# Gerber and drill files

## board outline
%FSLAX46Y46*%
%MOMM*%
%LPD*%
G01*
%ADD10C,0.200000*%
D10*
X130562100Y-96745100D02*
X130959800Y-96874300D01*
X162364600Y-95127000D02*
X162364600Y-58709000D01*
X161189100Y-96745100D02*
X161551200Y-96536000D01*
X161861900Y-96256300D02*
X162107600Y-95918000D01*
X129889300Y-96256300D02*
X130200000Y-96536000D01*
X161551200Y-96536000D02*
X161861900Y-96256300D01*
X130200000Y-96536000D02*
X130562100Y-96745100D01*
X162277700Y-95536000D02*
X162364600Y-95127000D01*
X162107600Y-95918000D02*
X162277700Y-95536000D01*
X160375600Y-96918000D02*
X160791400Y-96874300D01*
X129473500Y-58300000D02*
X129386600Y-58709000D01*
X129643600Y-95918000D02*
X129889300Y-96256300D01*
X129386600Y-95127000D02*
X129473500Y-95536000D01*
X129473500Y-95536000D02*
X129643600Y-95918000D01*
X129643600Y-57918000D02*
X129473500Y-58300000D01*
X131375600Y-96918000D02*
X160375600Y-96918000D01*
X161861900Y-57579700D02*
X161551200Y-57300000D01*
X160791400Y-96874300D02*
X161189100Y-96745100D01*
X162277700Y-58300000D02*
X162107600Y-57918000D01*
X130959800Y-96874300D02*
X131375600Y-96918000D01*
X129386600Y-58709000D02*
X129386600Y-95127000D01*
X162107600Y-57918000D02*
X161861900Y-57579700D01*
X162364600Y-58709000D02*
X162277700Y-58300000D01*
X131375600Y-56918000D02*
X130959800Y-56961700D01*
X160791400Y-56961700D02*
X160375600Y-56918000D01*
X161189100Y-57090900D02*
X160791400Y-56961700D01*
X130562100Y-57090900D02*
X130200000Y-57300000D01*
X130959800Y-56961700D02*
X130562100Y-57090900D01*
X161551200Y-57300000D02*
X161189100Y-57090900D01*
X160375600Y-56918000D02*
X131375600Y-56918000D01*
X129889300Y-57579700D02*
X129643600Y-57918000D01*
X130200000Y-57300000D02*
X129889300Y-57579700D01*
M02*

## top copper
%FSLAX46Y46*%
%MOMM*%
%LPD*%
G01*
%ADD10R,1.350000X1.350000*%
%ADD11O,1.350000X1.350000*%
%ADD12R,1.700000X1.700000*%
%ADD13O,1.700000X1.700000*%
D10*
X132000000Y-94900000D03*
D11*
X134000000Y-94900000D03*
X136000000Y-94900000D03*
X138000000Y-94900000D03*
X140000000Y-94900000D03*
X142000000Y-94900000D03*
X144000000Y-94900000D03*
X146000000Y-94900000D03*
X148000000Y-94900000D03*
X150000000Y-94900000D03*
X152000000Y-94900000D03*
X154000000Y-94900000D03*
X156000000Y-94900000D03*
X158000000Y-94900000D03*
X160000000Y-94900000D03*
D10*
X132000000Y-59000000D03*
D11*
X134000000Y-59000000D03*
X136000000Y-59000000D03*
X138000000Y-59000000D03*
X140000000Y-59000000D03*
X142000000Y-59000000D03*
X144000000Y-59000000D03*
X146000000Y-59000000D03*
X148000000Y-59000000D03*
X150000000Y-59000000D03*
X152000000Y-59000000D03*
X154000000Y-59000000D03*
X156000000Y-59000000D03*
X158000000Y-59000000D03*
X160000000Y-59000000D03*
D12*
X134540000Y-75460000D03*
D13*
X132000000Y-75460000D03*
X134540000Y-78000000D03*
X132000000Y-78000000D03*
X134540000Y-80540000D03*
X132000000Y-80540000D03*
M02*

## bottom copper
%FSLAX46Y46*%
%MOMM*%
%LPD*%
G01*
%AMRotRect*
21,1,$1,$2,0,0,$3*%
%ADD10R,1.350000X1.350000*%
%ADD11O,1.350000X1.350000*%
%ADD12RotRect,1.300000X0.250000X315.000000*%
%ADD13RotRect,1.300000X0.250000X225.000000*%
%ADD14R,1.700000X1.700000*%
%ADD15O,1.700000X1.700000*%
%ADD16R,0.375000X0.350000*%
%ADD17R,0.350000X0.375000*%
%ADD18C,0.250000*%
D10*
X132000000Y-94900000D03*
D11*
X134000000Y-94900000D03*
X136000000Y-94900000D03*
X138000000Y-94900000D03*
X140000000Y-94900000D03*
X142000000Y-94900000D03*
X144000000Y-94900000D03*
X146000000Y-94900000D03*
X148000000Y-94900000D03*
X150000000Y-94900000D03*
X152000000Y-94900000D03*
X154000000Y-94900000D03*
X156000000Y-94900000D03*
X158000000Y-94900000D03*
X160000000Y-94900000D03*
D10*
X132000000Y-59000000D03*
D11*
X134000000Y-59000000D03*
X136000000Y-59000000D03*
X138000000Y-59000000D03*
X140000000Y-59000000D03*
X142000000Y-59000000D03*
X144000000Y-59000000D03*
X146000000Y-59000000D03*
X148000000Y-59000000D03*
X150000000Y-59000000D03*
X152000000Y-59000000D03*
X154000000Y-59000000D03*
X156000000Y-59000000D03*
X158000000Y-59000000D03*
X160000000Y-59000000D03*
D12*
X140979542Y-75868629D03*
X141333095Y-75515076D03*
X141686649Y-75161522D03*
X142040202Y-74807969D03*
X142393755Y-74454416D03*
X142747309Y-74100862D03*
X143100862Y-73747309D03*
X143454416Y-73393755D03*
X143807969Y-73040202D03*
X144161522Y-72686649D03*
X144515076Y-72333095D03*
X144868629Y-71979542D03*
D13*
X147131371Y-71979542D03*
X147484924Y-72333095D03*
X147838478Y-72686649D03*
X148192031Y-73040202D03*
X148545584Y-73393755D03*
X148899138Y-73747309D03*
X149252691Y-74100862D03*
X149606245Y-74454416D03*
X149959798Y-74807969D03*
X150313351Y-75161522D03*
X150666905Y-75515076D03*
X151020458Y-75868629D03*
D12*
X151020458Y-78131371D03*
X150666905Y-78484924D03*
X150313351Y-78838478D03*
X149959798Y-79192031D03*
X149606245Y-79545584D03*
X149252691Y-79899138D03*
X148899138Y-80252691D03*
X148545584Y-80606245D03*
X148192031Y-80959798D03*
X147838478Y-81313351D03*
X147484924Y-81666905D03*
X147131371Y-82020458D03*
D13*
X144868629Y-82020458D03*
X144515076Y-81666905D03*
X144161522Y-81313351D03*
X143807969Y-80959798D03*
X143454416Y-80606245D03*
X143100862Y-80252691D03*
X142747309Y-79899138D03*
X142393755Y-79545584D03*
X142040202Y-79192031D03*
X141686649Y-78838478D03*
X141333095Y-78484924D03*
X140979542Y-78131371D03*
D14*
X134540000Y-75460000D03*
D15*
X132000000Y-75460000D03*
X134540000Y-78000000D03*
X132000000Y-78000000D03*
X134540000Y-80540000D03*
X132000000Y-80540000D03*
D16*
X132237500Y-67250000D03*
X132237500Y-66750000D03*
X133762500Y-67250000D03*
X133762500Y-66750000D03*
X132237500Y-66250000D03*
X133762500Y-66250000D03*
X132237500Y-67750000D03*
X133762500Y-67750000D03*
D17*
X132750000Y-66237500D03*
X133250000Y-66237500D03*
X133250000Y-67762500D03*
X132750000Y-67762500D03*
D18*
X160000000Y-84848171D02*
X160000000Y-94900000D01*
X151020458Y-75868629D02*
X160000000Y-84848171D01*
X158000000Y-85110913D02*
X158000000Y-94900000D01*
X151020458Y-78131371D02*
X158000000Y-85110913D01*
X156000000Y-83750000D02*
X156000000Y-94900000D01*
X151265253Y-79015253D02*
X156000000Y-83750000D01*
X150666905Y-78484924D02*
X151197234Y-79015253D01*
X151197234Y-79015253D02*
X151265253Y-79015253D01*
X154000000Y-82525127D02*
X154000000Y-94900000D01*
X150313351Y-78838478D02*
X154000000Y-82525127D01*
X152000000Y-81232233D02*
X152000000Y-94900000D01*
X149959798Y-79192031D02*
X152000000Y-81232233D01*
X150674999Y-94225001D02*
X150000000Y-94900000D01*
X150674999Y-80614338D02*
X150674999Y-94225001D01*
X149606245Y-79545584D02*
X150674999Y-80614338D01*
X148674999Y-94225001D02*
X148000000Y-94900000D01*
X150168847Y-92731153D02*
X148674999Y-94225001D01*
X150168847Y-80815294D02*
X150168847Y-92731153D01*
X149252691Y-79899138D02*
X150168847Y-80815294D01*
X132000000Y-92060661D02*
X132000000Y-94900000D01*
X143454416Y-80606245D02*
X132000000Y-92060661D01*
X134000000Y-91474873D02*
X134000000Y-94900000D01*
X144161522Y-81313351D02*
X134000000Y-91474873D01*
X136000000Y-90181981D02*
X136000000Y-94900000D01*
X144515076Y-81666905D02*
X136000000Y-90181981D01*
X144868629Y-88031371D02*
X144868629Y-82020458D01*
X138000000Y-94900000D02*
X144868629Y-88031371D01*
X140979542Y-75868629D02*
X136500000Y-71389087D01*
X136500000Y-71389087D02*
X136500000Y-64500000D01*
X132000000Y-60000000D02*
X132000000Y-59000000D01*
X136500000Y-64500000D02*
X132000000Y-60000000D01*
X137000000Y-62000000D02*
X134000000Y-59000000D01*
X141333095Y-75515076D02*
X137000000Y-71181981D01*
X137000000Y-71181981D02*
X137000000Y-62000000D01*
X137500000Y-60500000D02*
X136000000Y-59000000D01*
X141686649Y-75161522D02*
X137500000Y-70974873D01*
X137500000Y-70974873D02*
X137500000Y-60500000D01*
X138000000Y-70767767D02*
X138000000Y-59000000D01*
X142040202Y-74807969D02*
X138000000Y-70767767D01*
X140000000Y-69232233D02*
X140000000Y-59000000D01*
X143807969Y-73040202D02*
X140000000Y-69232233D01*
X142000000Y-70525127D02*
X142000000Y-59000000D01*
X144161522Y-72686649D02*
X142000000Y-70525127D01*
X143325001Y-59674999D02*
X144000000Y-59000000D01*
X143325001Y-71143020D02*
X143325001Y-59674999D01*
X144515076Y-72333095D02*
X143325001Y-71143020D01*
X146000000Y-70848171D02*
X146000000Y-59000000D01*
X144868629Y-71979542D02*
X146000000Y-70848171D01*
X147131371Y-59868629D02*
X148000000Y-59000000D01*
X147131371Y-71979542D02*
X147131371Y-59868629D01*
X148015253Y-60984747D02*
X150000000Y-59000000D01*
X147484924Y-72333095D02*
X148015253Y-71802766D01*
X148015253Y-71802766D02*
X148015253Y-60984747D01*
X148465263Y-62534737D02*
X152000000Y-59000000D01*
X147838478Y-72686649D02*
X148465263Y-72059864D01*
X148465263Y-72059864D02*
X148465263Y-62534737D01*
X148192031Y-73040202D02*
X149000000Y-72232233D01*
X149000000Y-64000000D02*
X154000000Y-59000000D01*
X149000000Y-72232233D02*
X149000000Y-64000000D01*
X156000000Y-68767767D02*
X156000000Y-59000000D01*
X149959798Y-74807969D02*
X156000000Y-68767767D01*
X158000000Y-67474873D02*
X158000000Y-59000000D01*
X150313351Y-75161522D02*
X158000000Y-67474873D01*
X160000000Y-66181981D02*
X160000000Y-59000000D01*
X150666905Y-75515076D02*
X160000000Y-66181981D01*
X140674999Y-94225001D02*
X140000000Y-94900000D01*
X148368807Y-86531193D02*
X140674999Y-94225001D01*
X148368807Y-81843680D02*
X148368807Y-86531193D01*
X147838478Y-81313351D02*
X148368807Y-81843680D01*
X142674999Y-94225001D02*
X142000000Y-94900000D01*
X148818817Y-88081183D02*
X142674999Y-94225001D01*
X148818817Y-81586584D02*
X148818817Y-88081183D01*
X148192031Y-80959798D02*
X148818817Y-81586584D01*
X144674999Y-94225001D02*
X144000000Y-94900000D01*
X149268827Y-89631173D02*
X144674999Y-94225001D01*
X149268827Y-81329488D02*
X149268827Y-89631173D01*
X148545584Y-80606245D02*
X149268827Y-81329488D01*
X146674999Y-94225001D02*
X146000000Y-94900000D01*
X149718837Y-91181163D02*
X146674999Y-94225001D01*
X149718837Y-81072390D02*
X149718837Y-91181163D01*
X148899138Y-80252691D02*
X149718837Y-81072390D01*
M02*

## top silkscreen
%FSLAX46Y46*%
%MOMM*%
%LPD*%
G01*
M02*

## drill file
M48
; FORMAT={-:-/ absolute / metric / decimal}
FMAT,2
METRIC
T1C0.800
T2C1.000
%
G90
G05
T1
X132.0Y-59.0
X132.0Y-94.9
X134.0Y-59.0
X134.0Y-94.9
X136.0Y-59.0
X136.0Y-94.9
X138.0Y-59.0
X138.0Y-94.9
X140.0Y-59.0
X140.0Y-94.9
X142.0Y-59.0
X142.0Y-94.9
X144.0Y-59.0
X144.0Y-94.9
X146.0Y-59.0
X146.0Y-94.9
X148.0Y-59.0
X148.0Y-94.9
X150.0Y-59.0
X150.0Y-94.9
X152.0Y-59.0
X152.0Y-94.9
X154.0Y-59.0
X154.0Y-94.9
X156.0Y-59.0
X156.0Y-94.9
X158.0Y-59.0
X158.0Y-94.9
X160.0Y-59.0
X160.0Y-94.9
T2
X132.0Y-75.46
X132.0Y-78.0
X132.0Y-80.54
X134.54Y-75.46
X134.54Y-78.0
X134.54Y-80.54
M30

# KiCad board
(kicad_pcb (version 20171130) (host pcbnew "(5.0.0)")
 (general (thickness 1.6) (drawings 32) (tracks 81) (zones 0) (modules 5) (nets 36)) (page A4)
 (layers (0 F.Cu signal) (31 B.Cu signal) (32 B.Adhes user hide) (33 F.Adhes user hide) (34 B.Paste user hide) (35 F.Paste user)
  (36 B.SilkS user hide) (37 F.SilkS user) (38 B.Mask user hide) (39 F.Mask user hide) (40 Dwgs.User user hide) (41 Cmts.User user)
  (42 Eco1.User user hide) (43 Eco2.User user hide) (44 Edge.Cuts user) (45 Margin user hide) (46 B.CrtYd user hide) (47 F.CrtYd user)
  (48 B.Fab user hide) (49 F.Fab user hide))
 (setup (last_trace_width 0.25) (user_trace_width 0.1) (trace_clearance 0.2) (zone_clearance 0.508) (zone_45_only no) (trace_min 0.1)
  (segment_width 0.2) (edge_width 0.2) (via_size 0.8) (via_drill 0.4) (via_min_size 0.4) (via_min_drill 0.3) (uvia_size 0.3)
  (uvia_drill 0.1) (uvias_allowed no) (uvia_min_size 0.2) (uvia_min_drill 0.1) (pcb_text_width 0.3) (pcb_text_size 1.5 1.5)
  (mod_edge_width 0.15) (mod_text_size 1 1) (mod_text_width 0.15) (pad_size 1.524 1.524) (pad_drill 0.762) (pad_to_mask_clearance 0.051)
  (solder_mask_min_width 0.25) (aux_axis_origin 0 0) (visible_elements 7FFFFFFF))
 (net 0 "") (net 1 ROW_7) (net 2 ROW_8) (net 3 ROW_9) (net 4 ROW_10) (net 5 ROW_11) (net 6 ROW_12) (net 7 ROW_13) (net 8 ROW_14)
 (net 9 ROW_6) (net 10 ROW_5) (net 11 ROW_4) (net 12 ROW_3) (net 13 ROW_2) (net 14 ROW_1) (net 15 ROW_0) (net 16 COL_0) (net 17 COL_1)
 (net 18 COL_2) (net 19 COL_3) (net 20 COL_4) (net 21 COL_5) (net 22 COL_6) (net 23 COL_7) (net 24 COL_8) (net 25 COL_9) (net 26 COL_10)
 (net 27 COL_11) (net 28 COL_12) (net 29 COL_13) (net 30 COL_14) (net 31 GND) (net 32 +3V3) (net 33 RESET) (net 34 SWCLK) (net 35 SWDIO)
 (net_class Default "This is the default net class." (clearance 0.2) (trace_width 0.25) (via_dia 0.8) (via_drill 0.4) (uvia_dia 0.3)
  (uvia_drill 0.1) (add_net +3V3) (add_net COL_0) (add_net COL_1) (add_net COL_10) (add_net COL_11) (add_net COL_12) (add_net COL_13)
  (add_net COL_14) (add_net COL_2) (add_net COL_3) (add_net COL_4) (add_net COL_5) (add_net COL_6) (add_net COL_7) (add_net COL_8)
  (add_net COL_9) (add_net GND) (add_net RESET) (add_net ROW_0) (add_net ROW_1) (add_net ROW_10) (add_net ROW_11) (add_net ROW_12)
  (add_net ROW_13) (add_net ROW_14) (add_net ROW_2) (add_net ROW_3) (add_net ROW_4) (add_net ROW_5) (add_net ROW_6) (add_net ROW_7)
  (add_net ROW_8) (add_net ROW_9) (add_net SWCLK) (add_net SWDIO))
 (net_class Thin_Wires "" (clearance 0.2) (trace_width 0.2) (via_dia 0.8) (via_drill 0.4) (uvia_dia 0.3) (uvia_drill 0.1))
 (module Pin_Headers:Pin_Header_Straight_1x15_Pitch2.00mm (layer F.Cu) (at 132 94.9 90)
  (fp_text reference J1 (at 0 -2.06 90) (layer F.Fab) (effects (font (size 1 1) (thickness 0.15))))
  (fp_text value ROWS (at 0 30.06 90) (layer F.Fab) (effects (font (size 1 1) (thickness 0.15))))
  (pad 1 thru_hole rect (at 0 0 90) (size 1.35 1.35) (drill 0.8) (layers *.Cu *.Mask) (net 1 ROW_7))
  (pad 2 thru_hole oval (at 0 2 90) (size 1.35 1.35) (drill 0.8) (layers *.Cu *.Mask) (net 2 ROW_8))
  (pad 3 thru_hole oval (at 0 4 90) (size 1.35 1.35) (drill 0.8) (layers *.Cu *.Mask) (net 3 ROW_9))
  (pad 4 thru_hole oval (at 0 6 90) (size 1.35 1.35) (drill 0.8) (layers *.Cu *.Mask) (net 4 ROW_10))
  (pad 5 thru_hole oval (at 0 8 90) (size 1.35 1.35) (drill 0.8) (layers *.Cu *.Mask) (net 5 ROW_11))
  (pad 6 thru_hole oval (at 0 10 90) (size 1.35 1.35) (drill 0.8) (layers *.Cu *.Mask) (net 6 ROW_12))
  (pad 7 thru_hole oval (at 0 12 90) (size 1.35 1.35) (drill 0.8) (layers *.Cu *.Mask) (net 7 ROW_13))
  (pad 8 thru_hole oval (at 0 14 90) (size 1.35 1.35) (drill 0.8) (layers *.Cu *.Mask) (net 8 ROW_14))
  (pad 9 thru_hole oval (at 0 16 90) (size 1.35 1.35) (drill 0.8) (layers *.Cu *.Mask) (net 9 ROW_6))
  (pad 10 thru_hole oval (at 0 18 90) (size 1.35 1.35) (drill 0.8) (layers *.Cu *.Mask) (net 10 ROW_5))
  (pad 11 thru_hole oval (at 0 20 90) (size 1.35 1.35) (drill 0.8) (layers *.Cu *.Mask) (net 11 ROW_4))
  (pad 12 thru_hole oval (at 0 22 90) (size 1.35 1.35) (drill 0.8) (layers *.Cu *.Mask) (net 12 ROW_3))
  (pad 13 thru_hole oval (at 0 24 90) (size 1.35 1.35) (drill 0.8) (layers *.Cu *.Mask) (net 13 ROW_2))
  (pad 14 thru_hole oval (at 0 26 90) (size 1.35 1.35) (drill 0.8) (layers *.Cu *.Mask) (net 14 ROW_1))
  (pad 15 thru_hole oval (at 0 28 90) (size 1.35 1.35) (drill 0.8) (layers *.Cu *.Mask) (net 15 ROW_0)))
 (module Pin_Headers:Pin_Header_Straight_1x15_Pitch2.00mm (layer F.Cu) (at 132 59 90)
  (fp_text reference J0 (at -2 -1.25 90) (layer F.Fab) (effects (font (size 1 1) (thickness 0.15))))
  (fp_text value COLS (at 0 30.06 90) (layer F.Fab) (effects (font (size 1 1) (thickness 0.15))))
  (pad 1 thru_hole rect (at 0 0 90) (size 1.35 1.35) (drill 0.8) (layers *.Cu *.Mask) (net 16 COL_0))
  (pad 2 thru_hole oval (at 0 2 90) (size 1.35 1.35) (drill 0.8) (layers *.Cu *.Mask) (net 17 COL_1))
  (pad 3 thru_hole oval (at 0 4 90) (size 1.35 1.35) (drill 0.8) (layers *.Cu *.Mask) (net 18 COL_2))
  (pad 4 thru_hole oval (at 0 6 90) (size 1.35 1.35) (drill 0.8) (layers *.Cu *.Mask) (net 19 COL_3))
  (pad 5 thru_hole oval (at 0 8 90) (size 1.35 1.35) (drill 0.8) (layers *.Cu *.Mask) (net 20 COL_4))
  (pad 6 thru_hole oval (at 0 10 90) (size 1.35 1.35) (drill 0.8) (layers *.Cu *.Mask) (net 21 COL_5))
  (pad 7 thru_hole oval (at 0 12 90) (size 1.35 1.35) (drill 0.8) (layers *.Cu *.Mask) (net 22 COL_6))
  (pad 8 thru_hole oval (at 0 14 90) (size 1.35 1.35) (drill 0.8) (layers *.Cu *.Mask) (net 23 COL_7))
  (pad 9 thru_hole oval (at 0 16 90) (size 1.35 1.35) (drill 0.8) (layers *.Cu *.Mask) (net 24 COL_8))
  (pad 10 thru_hole oval (at 0 18 90) (size 1.35 1.35) (drill 0.8) (layers *.Cu *.Mask) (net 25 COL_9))
  (pad 11 thru_hole oval (at 0 20 90) (size 1.35 1.35) (drill 0.8) (layers *.Cu *.Mask) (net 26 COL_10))
  (pad 12 thru_hole oval (at 0 22 90) (size 1.35 1.35) (drill 0.8) (layers *.Cu *.Mask) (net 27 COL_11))
  (pad 13 thru_hole oval (at 0 24 90) (size 1.35 1.35) (drill 0.8) (layers *.Cu *.Mask) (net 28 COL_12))
  (pad 14 thru_hole oval (at 0 26 90) (size 1.35 1.35) (drill 0.8) (layers *.Cu *.Mask) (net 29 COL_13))
  (pad 15 thru_hole oval (at 0 28 90) (size 1.35 1.35) (drill 0.8) (layers *.Cu *.Mask) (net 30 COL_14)))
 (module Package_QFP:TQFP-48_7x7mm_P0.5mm (layer B.Cu) (at 146 77 315)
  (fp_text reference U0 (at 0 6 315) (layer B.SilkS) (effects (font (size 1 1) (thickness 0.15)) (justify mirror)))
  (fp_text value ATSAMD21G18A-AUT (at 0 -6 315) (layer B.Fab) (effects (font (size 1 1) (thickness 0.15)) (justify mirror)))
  (pad 1 smd rect (at -4.35 2.75 315) (size 1.3 0.25) (layers B.Cu B.Paste B.Mask) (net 16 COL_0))
  (pad 2 smd rect (at -4.35 2.25 315) (size 1.3 0.25) (layers B.Cu B.Paste B.Mask) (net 17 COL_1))
  (pad 3 smd rect (at -4.35 1.749999 315) (size 1.3 0.25) (layers B.Cu B.Paste B.Mask) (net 18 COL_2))
  (pad 4 smd rect (at -4.35 1.25 315) (size 1.3 0.25) (layers B.Cu B.Paste B.Mask) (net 19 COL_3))
  (pad 5 smd rect (at -4.35 0.750001 315) (size 1.3 0.25) (layers B.Cu B.Paste B.Mask) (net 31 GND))
  (pad 6 smd rect (at -4.35 0.25 315) (size 1.3 0.25) (layers B.Cu B.Paste B.Mask) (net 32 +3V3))
  (pad 7 smd rect (at -4.35 -0.25 315) (size 1.3 0.25) (layers B.Cu B.Paste B.Mask))
  (pad 8 smd rect (at -4.35 -0.750001 315) (size 1.3 0.25) (layers B.Cu B.Paste B.Mask))
  (pad 9 smd rect (at -4.35 -1.25 315) (size 1.3 0.25) (layers B.Cu B.Paste B.Mask) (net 20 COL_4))
  (pad 10 smd rect (at -4.35 -1.749999 315) (size 1.3 0.25) (layers B.Cu B.Paste B.Mask) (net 21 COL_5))
  (pad 11 smd rect (at -4.35 -2.25 315) (size 1.3 0.25) (layers B.Cu B.Paste B.Mask) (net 22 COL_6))
  (pad 12 smd rect (at -4.35 -2.75 315) (size 1.3 0.25) (layers B.Cu B.Paste B.Mask) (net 23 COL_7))
  (pad 13 smd rect (at -2.75 -4.35 225) (size 1.3 0.25) (layers B.Cu B.Paste B.Mask) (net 24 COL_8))
  (pad 14 smd rect (at -2.25 -4.35 225) (size 1.3 0.25) (layers B.Cu B.Paste B.Mask) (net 25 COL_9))
  (pad 15 smd rect (at -1.749999 -4.35 225) (size 1.3 0.25) (layers B.Cu B.Paste B.Mask) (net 26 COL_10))
  (pad 16 smd rect (at -1.25 -4.35 225) (size 1.3 0.25) (layers B.Cu B.Paste B.Mask) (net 27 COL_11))
  (pad 17 smd rect (at -0.750001 -4.35 225) (size 1.3 0.25) (layers B.Cu B.Paste B.Mask) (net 32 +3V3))
  (pad 18 smd rect (at -0.25 -4.35 225) (size 1.3 0.25) (layers B.Cu B.Paste B.Mask) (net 31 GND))
  (pad 19 smd rect (at 0.25 -4.35 225) (size 1.3 0.25) (layers B.Cu B.Paste B.Mask))
  (pad 20 smd rect (at 0.750001 -4.35 225) (size 1.3 0.25) (layers B.Cu B.Paste B.Mask))
  (pad 21 smd rect (at 1.25 -4.35 225) (size 1.3 0.25) (layers B.Cu B.Paste B.Mask) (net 28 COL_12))
  (pad 22 smd rect (at 1.749999 -4.35 225) (size 1.3 0.25) (layers B.Cu B.Paste B.Mask) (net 29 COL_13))
  (pad 23 smd rect (at 2.25 -4.35 225) (size 1.3 0.25) (layers B.Cu B.Paste B.Mask) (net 30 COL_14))
  (pad 24 smd rect (at 2.75 -4.35 225) (size 1.3 0.25) (layers B.Cu B.Paste B.Mask) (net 15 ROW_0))
  (pad 25 smd rect (at 4.35 -2.75 315) (size 1.3 0.25) (layers B.Cu B.Paste B.Mask) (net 14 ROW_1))
  (pad 26 smd rect (at 4.35 -2.25 315) (size 1.3 0.25) (layers B.Cu B.Paste B.Mask) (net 13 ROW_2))
  (pad 27 smd rect (at 4.35 -1.749999 315) (size 1.3 0.25) (layers B.Cu B.Paste B.Mask) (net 12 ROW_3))
  (pad 28 smd rect (at 4.35 -1.25 315) (size 1.3 0.25) (layers B.Cu B.Paste B.Mask) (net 11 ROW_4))
  (pad 29 smd rect (at 4.35 -0.750001 315) (size 1.3 0.25) (layers B.Cu B.Paste B.Mask) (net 10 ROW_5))
  (pad 30 smd rect (at 4.35 -0.25 315) (size 1.3 0.25) (layers B.Cu B.Paste B.Mask) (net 9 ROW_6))
  (pad 31 smd rect (at 4.35 0.25 315) (size 1.3 0.25) (layers B.Cu B.Paste B.Mask) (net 8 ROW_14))
  (pad 32 smd rect (at 4.35 0.750001 315) (size 1.3 0.25) (layers B.Cu B.Paste B.Mask) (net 7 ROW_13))
  (pad 33 smd rect (at 4.35 1.25 315) (size 1.3 0.25) (layers B.Cu B.Paste B.Mask) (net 6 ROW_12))
  (pad 34 smd rect (at 4.35 1.749999 315) (size 1.3 0.25) (layers B.Cu B.Paste B.Mask) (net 5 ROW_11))
  (pad 35 smd rect (at 4.35 2.25 315) (size 1.3 0.25) (layers B.Cu B.Paste B.Mask) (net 31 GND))
  (pad 36 smd rect (at 4.35 2.75 315) (size 1.3 0.25) (layers B.Cu B.Paste B.Mask) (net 32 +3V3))
  (pad 37 smd rect (at 2.75 4.35 225) (size 1.3 0.25) (layers B.Cu B.Paste B.Mask) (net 4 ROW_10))
  (pad 38 smd rect (at 2.25 4.35 225) (size 1.3 0.25) (layers B.Cu B.Paste B.Mask) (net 3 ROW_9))
  (pad 39 smd rect (at 1.749999 4.35 225) (size 1.3 0.25) (layers B.Cu B.Paste B.Mask) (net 2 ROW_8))
  (pad 40 smd rect (at 1.25 4.35 225) (size 1.3 0.25) (layers B.Cu B.Paste B.Mask) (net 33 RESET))
  (pad 41 smd rect (at 0.750001 4.35 225) (size 1.3 0.25) (layers B.Cu B.Paste B.Mask) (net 1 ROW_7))
  (pad 42 smd rect (at 0.25 4.35 225) (size 1.3 0.25) (layers B.Cu B.Paste B.Mask) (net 31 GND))
  (pad 43 smd rect (at -0.25 4.35 225) (size 1.3 0.25) (layers B.Cu B.Paste B.Mask) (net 32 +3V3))
  (pad 44 smd rect (at -0.750001 4.35 225) (size 1.3 0.25) (layers B.Cu B.Paste B.Mask) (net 32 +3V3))
  (pad 45 smd rect (at -1.25 4.35 225) (size 1.3 0.25) (layers B.Cu B.Paste B.Mask) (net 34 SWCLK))
  (pad 46 smd rect (at -1.749999 4.35 225) (size 1.3 0.25) (layers B.Cu B.Paste B.Mask) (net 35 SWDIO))
  (pad 47 smd rect (at -2.25 4.35 225) (size 1.3 0.25) (layers B.Cu B.Paste B.Mask))
  (pad 48 smd rect (at -2.75 4.35 225) (size 1.3 0.25) (layers B.Cu B.Paste B.Mask)))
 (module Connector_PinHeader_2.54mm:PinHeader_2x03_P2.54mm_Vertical (layer B.Cu) (at 134.54 75.46 180)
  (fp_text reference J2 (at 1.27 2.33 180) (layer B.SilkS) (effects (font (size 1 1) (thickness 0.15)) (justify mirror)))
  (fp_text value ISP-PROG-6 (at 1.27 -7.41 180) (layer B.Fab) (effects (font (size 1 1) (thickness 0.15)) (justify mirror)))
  (pad 1 thru_hole rect (at 0 0 180) (size 1.7 1.7) (drill 1) (layers *.Cu *.Mask) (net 35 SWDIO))
  (pad 2 thru_hole oval (at 2.54 0 180) (size 1.7 1.7) (drill 1) (layers *.Cu *.Mask) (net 32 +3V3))
  (pad 3 thru_hole oval (at 0 -2.54 180) (size 1.7 1.7) (drill 1) (layers *.Cu *.Mask) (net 34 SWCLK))
  (pad 4 thru_hole oval (at 2.54 -2.54 180) (size 1.7 1.7) (drill 1) (layers *.Cu *.Mask))
  (pad 5 thru_hole oval (at 0 -5.08 180) (size 1.7 1.7) (drill 1) (layers *.Cu *.Mask) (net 33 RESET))
  (pad 6 thru_hole oval (at 2.54 -5.08 180) (size 1.7 1.7) (drill 1) (layers *.Cu *.Mask) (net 31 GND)))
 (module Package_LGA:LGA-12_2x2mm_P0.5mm (layer B.Cu) (at 133 67)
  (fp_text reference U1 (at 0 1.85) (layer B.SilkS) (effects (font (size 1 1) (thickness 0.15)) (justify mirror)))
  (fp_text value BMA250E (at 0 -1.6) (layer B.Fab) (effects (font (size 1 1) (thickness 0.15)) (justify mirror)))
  (pad 2 smd rect (at -0.7625 0.25) (size 0.375 0.35) (layers B.Cu B.Paste B.Mask))
  (pad 3 smd rect (at -0.7625 -0.25) (size 0.375 0.35) (layers B.Cu B.Paste B.Mask))
  (pad 9 smd rect (at 0.7625 0.25) (size 0.375 0.35) (layers B.Cu B.Paste B.Mask))
  (pad 8 smd rect (at 0.7625 -0.25) (size 0.375 0.35) (layers B.Cu B.Paste B.Mask))
  (pad 4 smd rect (at -0.7625 -0.75) (size 0.375 0.35) (layers B.Cu B.Paste B.Mask))
  (pad 7 smd rect (at 0.7625 -0.75) (size 0.375 0.35) (layers B.Cu B.Paste B.Mask))
  (pad 1 smd rect (at -0.7625 0.75) (size 0.375 0.35) (layers B.Cu B.Paste B.Mask))
  (pad 10 smd rect (at 0.7625 0.75) (size 0.375 0.35) (layers B.Cu B.Paste B.Mask))
  (pad 5 smd rect (at -0.25 -0.7625 270) (size 0.375 0.35) (layers B.Cu B.Paste B.Mask))
  (pad 6 smd rect (at 0.25 -0.7625 270) (size 0.375 0.35) (layers B.Cu B.Paste B.Mask))
  (pad 11 smd rect (at 0.25 0.7625 270) (size 0.375 0.35) (layers B.Cu B.Paste B.Mask))
  (pad 12 smd rect (at -0.25 0.7625 270) (size 0.375 0.35) (layers B.Cu B.Paste B.Mask)))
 (gr_line (start 130.5621 96.7451) (end 130.9598 96.8743) (layer Edge.Cuts) (width 0.2))
 (gr_line (start 162.3646 95.127) (end 162.3646 58.709) (layer Edge.Cuts) (width 0.2))
 (gr_line (start 161.1891 96.7451) (end 161.5512 96.536) (layer Edge.Cuts) (width 0.2))
 (gr_line (start 161.8619 96.2563) (end 162.1076 95.918) (layer Edge.Cuts) (width 0.2))
 (gr_line (start 129.8893 96.2563) (end 130.2 96.536) (layer Edge.Cuts) (width 0.2))
 (gr_line (start 161.5512 96.536) (end 161.8619 96.2563) (layer Edge.Cuts) (width 0.2))
 (gr_line (start 130.2 96.536) (end 130.5621 96.7451) (layer Edge.Cuts) (width 0.2))
 (gr_line (start 162.2777 95.536) (end 162.3646 95.127) (layer Edge.Cuts) (width 0.2))
 (gr_line (start 162.1076 95.918) (end 162.2777 95.536) (layer Edge.Cuts) (width 0.2))
 (gr_line (start 160.3756 96.918) (end 160.7914 96.8743) (layer Edge.Cuts) (width 0.2))
 (gr_line (start 129.4735 58.3) (end 129.3866 58.709) (layer Edge.Cuts) (width 0.2))
 (gr_line (start 129.6436 95.918) (end 129.8893 96.2563) (layer Edge.Cuts) (width 0.2))
 (gr_line (start 129.3866 95.127) (end 129.4735 95.536) (layer Edge.Cuts) (width 0.2))
 (gr_line (start 129.4735 95.536) (end 129.6436 95.918) (layer Edge.Cuts) (width 0.2))
 (gr_line (start 129.6436 57.918) (end 129.4735 58.3) (layer Edge.Cuts) (width 0.2))
 (gr_line (start 131.3756 96.918) (end 160.3756 96.918) (layer Edge.Cuts) (width 0.2))
 (gr_line (start 161.8619 57.5797) (end 161.5512 57.3) (layer Edge.Cuts) (width 0.2))
 (gr_line (start 160.7914 96.8743) (end 161.1891 96.7451) (layer Edge.Cuts) (width 0.2))
 (gr_line (start 162.2777 58.3) (end 162.1076 57.918) (layer Edge.Cuts) (width 0.2))
 (gr_line (start 130.9598 96.8743) (end 131.3756 96.918) (layer Edge.Cuts) (width 0.2))
 (gr_line (start 129.3866 58.709) (end 129.3866 95.127) (layer Edge.Cuts) (width 0.2))
 (gr_line (start 162.1076 57.918) (end 161.8619 57.5797) (layer Edge.Cuts) (width 0.2))
 (gr_line (start 162.3646 58.709) (end 162.2777 58.3) (layer Edge.Cuts) (width 0.2))
 (gr_line (start 131.3756 56.918) (end 130.9598 56.9617) (layer Edge.Cuts) (width 0.2))
 (gr_line (start 160.7914 56.9617) (end 160.3756 56.918) (layer Edge.Cuts) (width 0.2))
 (gr_line (start 161.1891 57.0909) (end 160.7914 56.9617) (layer Edge.Cuts) (width 0.2))
 (gr_line (start 130.5621 57.0909) (end 130.2 57.3) (layer Edge.Cuts) (width 0.2))
 (gr_line (start 130.9598 56.9617) (end 130.5621 57.0909) (layer Edge.Cuts) (width 0.2))
 (gr_line (start 161.5512 57.3) (end 161.1891 57.0909) (layer Edge.Cuts) (width 0.2))
 (gr_line (start 160.3756 56.918) (end 131.3756 56.918) (layer Edge.Cuts) (width 0.2))
 (gr_line (start 129.8893 57.5797) (end 129.6436 57.918) (layer Edge.Cuts) (width 0.2))
 (gr_line (start 130.2 57.3) (end 129.8893 57.5797) (layer Edge.Cuts) (width 0.2))
 (segment (start 160 84.848171) (end 160 94.9) (width 0.25) (layer B.Cu) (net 15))
 (segment (start 151.020458 75.868629) (end 160 84.848171) (width 0.25) (layer B.Cu) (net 15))
 (segment (start 158 85.110913) (end 158 94.9) (width 0.25) (layer B.Cu) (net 14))
 (segment (start 151.020458 78.131371) (end 158 85.110913) (width 0.25) (layer B.Cu) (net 14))
 (segment (start 156 83.75) (end 156 94.9) (width 0.25) (layer B.Cu) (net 13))
 (segment (start 151.265253 79.015253) (end 156 83.75) (width 0.25) (layer B.Cu) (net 13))
 (segment (start 150.666905 78.484924) (end 151.197234 79.015253) (width 0.25) (layer B.Cu) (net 13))
 (segment (start 151.197234 79.015253) (end 151.265253 79.015253) (width 0.25) (layer B.Cu) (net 13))
 (segment (start 154 82.525127) (end 154 94.9) (width 0.25) (layer B.Cu) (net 12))
 (segment (start 150.313351 78.838478) (end 154 82.525127) (width 0.25) (layer B.Cu) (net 12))
 (segment (start 152 81.232233) (end 152 94.9) (width 0.25) (layer B.Cu) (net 11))
 (segment (start 149.959798 79.192031) (end 152 81.232233) (width 0.25) (layer B.Cu) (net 11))
 (segment (start 150.674999 94.225001) (end 150 94.9) (width 0.25) (layer B.Cu) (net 10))
 (segment (start 150.674999 80.614338) (end 150.674999 94.225001) (width 0.25) (layer B.Cu) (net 10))
 (segment (start 149.606245 79.545584) (end 150.674999 80.614338) (width 0.25) (layer B.Cu) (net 10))
 (segment (start 148.674999 94.225001) (end 148 94.9) (width 0.25) (layer B.Cu) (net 9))
 (segment (start 150.168847 92.731153) (end 148.674999 94.225001) (width 0.25) (layer B.Cu) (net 9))
 (segment (start 150.168847 80.815294) (end 150.168847 92.731153) (width 0.25) (layer B.Cu) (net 9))
 (segment (start 149.252691 79.899138) (end 150.168847 80.815294) (width 0.25) (layer B.Cu) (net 9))
 (segment (start 132 92.060661) (end 132 94.9) (width 0.25) (layer B.Cu) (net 1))
 (segment (start 143.454416 80.606245) (end 132 92.060661) (width 0.25) (layer B.Cu) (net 1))
 (segment (start 134 91.474873) (end 134 94.9) (width 0.25) (layer B.Cu) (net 2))
 (segment (start 144.161522 81.313351) (end 134 91.474873) (width 0.25) (layer B.Cu) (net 2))
 (segment (start 136 90.181981) (end 136 94.9) (width 0.25) (layer B.Cu) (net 3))
 (segment (start 144.515076 81.666905) (end 136 90.181981) (width 0.25) (layer B.Cu) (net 3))
 (segment (start 144.868629 88.031371) (end 144.868629 82.020458) (width 0.25) (layer B.Cu) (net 4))
 (segment (start 138 94.9) (end 144.868629 88.031371) (width 0.25) (layer B.Cu) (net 4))
 (segment (start 140.979542 75.868629) (end 136.5 71.389087) (width 0.25) (layer B.Cu) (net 16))
 (segment (start 136.5 71.389087) (end 136.5 64.5) (width 0.25) (layer B.Cu) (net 16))
 (segment (start 132 60) (end 132 59) (width 0.25) (layer B.Cu) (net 16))
 (segment (start 136.5 64.5) (end 132 60) (width 0.25) (layer B.Cu) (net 16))
 (segment (start 137 62) (end 134 59) (width 0.25) (layer B.Cu) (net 17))
 (segment (start 141.333095 75.515076) (end 137 71.181981) (width 0.25) (layer B.Cu) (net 17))
 (segment (start 137 71.181981) (end 137 62) (width 0.25) (layer B.Cu) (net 17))
 (segment (start 137.5 60.5) (end 136 59) (width 0.25) (layer B.Cu) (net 18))
 (segment (start 141.686649 75.161522) (end 137.5 70.974873) (width 0.25) (layer B.Cu) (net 18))
 (segment (start 137.5 70.974873) (end 137.5 60.5) (width 0.25) (layer B.Cu) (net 18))
 (segment (start 138 70.767767) (end 138 59) (width 0.25) (layer B.Cu) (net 19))
 (segment (start 142.040202 74.807969) (end 138 70.767767) (width 0.25) (layer B.Cu) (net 19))
 (segment (start 140 69.232233) (end 140 59) (width 0.25) (layer B.Cu) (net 20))
 (segment (start 143.807969 73.040202) (end 140 69.232233) (width 0.25) (layer B.Cu) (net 20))
 (segment (start 142 70.525127) (end 142 59) (width 0.25) (layer B.Cu) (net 21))
 (segment (start 144.161522 72.686649) (end 142 70.525127) (width 0.25) (layer B.Cu) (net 21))
 (segment (start 143.325001 59.674999) (end 144 59) (width 0.25) (layer B.Cu) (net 22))
 (segment (start 143.325001 71.14302) (end 143.325001 59.674999) (width 0.25) (layer B.Cu) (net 22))
 (segment (start 144.515076 72.333095) (end 143.325001 71.14302) (width 0.25) (layer B.Cu) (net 22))
 (segment (start 146 70.848171) (end 146 59) (width 0.25) (layer B.Cu) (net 23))
 (segment (start 144.868629 71.979542) (end 146 70.848171) (width 0.25) (layer B.Cu) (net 23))
 (segment (start 147.131371 59.868629) (end 148 59) (width 0.25) (layer B.Cu) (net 24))
 (segment (start 147.131371 71.979542) (end 147.131371 59.868629) (width 0.25) (layer B.Cu) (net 24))
 (segment (start 148.015253 60.984747) (end 150 59) (width 0.25) (layer B.Cu) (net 25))
 (segment (start 147.484924 72.333095) (end 148.015253 71.802766) (width 0.25) (layer B.Cu) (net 25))
 (segment (start 148.015253 71.802766) (end 148.015253 60.984747) (width 0.25) (layer B.Cu) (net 25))
 (segment (start 148.465263 62.534737) (end 152 59) (width 0.25) (layer B.Cu) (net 26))
 (segment (start 147.838478 72.686649) (end 148.465263 72.059864) (width 0.25) (layer B.Cu) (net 26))
 (segment (start 148.465263 72.059864) (end 148.465263 62.534737) (width 0.25) (layer B.Cu) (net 26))
 (segment (start 148.192031 73.040202) (end 149 72.232233) (width 0.25) (layer B.Cu) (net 27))
 (segment (start 149 64) (end 154 59) (width 0.25) (layer B.Cu) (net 27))
 (segment (start 149 72.232233) (end 149 64) (width 0.25) (layer B.Cu) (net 27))
 (segment (start 156 68.767767) (end 156 59) (width 0.25) (layer B.Cu) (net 28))
 (segment (start 149.959798 74.807969) (end 156 68.767767) (width 0.25) (layer B.Cu) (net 28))
 (segment (start 158 67.474873) (end 158 59) (width 0.25) (layer B.Cu) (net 29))
 (segment (start 150.313351 75.161522) (end 158 67.474873) (width 0.25) (layer B.Cu) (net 29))
 (segment (start 160 66.181981) (end 160 59) (width 0.25) (layer B.Cu) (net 30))
 (segment (start 150.666905 75.515076) (end 160 66.181981) (width 0.25) (layer B.Cu) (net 30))
 (segment (start 140.674999 94.225001) (end 140 94.9) (width 0.25) (layer B.Cu) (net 5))
 (segment (start 148.368807 86.531193) (end 140.674999 94.225001) (width 0.25) (layer B.Cu) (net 5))
 (segment (start 148.368807 81.84368) (end 148.368807 86.531193) (width 0.25) (layer B.Cu) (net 5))
 (segment (start 147.838478 81.313351) (end 148.368807 81.84368) (width 0.25) (layer B.Cu) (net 5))
 (segment (start 142.674999 94.225001) (end 142 94.9) (width 0.25) (layer B.Cu) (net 6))
 (segment (start 148.818817 88.081183) (end 142.674999 94.225001) (width 0.25) (layer B.Cu) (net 6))
 (segment (start 148.818817 81.586584) (end 148.818817 88.081183) (width 0.25) (layer B.Cu) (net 6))
 (segment (start 148.192031 80.959798) (end 148.818817 81.586584) (width 0.25) (layer B.Cu) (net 6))
 (segment (start 144.674999 94.225001) (end 144 94.9) (width 0.25) (layer B.Cu) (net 7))
 (segment (start 149.268827 89.631173) (end 144.674999 94.225001) (width 0.25) (layer B.Cu) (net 7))
 (segment (start 149.268827 81.329488) (end 149.268827 89.631173) (width 0.25) (layer B.Cu) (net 7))
 (segment (start 148.545584 80.606245) (end 149.268827 81.329488) (width 0.25) (layer B.Cu) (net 7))
 (segment (start 146.674999 94.225001) (end 146 94.9) (width 0.25) (layer B.Cu) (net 8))
 (segment (start 149.718837 91.181163) (end 146.674999 94.225001) (width 0.25) (layer B.Cu) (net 8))
 (segment (start 149.718837 81.07239) (end 149.718837 91.181163) (width 0.25) (layer B.Cu) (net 8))
 (segment (start 148.899138 80.252691) (end 149.718837 81.07239) (width 0.25) (layer B.Cu) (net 8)))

